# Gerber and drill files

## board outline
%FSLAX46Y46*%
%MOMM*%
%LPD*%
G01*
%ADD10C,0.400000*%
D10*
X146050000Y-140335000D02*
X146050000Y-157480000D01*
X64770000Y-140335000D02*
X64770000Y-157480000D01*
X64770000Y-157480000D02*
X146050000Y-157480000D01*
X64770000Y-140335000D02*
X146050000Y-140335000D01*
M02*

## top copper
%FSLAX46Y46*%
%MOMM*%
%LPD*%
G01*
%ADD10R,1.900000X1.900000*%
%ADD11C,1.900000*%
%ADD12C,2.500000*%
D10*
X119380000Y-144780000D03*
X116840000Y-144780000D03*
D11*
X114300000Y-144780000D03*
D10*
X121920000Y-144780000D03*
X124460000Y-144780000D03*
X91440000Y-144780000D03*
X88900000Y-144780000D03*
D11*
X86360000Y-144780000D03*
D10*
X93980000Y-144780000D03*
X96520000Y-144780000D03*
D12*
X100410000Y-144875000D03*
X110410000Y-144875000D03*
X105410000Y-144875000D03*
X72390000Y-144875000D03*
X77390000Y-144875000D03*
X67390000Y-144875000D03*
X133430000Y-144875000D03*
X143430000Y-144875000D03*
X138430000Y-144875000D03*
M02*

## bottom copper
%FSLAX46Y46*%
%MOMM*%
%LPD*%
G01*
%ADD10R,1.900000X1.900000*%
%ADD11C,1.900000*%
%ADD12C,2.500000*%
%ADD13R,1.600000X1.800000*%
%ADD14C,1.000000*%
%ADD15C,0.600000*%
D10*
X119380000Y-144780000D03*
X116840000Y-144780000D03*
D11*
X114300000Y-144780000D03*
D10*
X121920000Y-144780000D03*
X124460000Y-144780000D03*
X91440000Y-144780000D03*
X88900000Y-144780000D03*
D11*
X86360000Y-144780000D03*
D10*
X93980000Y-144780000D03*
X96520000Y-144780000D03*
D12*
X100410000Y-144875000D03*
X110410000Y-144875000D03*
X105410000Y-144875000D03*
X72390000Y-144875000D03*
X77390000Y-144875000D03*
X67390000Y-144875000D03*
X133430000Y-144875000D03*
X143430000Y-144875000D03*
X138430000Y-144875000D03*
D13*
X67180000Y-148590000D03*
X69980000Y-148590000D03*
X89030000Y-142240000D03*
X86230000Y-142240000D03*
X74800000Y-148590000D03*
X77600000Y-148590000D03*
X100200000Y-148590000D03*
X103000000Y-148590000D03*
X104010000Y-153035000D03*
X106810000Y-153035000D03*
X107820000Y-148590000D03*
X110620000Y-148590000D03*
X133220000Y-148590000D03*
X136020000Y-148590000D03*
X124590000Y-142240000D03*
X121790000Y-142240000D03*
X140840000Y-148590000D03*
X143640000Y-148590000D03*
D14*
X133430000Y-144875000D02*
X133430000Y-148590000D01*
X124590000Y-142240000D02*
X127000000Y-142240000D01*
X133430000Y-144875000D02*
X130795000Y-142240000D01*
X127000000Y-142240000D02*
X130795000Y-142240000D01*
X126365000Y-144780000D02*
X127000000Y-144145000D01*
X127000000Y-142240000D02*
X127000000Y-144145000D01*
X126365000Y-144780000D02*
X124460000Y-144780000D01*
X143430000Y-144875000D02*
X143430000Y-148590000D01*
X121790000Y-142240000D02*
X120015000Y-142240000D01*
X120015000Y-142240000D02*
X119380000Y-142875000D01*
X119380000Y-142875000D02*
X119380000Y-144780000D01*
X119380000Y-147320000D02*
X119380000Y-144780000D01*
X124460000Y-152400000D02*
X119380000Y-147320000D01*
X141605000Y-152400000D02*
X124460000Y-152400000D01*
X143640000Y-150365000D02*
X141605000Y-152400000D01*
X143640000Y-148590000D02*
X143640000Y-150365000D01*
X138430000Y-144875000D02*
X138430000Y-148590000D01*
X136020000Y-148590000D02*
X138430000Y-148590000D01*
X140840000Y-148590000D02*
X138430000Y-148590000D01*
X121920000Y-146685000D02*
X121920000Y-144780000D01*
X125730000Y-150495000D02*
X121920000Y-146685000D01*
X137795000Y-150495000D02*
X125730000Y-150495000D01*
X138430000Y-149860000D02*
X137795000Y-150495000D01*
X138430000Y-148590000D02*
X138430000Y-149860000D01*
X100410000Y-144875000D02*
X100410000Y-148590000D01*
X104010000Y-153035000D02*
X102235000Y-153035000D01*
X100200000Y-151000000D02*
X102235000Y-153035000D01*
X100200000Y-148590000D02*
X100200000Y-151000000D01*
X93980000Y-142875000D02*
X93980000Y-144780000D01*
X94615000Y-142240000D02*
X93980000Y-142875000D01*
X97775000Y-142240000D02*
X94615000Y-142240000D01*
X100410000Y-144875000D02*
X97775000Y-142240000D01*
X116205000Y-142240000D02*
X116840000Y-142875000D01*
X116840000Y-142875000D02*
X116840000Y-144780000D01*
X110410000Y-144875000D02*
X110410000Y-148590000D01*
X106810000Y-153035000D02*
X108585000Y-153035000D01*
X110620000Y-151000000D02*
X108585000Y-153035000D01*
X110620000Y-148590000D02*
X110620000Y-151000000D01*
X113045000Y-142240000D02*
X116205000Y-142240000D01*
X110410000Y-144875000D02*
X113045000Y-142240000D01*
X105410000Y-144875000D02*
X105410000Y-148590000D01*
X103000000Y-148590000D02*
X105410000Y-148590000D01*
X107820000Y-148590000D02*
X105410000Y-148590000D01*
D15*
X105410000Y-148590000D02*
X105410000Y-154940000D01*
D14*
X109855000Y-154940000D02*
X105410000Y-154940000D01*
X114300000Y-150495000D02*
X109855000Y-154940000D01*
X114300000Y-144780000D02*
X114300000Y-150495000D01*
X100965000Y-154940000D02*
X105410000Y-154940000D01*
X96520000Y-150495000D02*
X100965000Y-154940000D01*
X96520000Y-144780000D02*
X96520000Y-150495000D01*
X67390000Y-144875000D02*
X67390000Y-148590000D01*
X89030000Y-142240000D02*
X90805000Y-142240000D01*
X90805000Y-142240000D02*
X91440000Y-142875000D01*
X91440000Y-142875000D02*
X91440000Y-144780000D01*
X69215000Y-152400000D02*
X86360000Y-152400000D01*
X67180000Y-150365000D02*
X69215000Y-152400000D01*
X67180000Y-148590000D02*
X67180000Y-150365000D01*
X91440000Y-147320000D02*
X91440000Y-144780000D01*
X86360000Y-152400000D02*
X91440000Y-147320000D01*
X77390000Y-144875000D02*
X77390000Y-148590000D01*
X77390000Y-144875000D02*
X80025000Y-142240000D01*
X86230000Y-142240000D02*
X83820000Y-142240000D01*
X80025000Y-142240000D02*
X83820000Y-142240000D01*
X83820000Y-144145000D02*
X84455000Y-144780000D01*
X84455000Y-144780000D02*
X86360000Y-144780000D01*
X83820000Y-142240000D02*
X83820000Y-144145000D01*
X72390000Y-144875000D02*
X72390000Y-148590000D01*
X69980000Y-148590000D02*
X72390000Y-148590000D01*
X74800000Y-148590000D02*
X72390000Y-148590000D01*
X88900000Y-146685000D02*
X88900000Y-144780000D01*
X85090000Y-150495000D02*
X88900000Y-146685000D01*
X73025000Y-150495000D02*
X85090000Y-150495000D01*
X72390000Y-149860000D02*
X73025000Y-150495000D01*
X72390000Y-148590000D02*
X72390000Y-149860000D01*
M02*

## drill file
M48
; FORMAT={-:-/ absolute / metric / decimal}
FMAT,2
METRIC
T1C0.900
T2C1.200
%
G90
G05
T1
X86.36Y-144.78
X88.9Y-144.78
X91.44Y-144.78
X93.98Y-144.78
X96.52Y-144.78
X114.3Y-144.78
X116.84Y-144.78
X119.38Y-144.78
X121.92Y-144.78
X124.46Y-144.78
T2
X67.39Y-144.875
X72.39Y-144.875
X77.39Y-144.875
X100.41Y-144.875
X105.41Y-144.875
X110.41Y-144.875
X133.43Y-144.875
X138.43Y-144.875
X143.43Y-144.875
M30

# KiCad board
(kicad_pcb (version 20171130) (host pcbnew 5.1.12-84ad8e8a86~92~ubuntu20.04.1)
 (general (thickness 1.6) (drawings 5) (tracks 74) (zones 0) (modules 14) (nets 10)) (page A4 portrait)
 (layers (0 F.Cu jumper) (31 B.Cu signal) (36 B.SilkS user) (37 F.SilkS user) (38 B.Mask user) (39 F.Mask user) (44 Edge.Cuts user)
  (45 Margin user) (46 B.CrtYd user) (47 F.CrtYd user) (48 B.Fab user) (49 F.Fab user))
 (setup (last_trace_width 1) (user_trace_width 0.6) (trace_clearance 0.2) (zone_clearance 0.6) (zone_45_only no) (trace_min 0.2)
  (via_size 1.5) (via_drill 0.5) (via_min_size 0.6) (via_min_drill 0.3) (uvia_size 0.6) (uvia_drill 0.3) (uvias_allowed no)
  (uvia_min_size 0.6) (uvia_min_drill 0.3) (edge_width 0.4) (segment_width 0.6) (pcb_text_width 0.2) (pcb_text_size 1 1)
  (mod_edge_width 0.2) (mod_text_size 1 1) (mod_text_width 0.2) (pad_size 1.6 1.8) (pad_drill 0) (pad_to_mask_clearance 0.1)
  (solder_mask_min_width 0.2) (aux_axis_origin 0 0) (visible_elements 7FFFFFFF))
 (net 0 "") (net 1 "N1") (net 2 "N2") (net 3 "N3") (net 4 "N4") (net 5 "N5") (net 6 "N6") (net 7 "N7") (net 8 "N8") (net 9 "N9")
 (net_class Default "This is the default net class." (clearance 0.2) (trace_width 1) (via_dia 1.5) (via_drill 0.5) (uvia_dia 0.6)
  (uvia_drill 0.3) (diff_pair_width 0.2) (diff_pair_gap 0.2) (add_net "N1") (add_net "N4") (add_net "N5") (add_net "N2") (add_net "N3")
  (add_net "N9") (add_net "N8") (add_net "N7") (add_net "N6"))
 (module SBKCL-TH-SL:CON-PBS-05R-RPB (layer F.Cu) (at 119.38 144.78)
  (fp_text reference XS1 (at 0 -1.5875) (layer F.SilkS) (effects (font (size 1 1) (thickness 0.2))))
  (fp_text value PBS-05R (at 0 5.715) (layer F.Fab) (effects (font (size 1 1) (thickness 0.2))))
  (pad 3 thru_hole rect (at 0 0) (size 1.9 1.9) (drill 0.9) (layers B.Cu B.Mask) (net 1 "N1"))
  (pad 2 thru_hole rect (at -2.54 0) (size 1.9 1.9) (drill 0.9) (layers B.Cu B.Mask) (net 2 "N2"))
  (pad 1 thru_hole circle (at -5.08 0) (size 1.9 1.9) (drill 0.9) (layers B.Cu B.Mask) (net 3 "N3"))
  (pad 4 thru_hole rect (at 2.54 0) (size 1.9 1.9) (drill 0.9) (layers B.Cu B.Mask) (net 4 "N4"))
  (pad 5 thru_hole rect (at 5.08 0) (size 1.9 1.9) (drill 0.9) (layers B.Cu B.Mask) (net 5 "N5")))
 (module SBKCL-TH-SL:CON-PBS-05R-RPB (layer F.Cu) (at 91.44 144.78)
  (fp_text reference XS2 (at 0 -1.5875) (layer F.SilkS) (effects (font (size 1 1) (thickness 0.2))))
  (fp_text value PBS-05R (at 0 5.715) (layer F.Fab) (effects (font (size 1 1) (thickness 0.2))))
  (pad 3 thru_hole rect (at 0 0) (size 1.9 1.9) (drill 0.9) (layers B.Cu B.Mask) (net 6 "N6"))
  (pad 2 thru_hole rect (at -2.54 0) (size 1.9 1.9) (drill 0.9) (layers B.Cu B.Mask) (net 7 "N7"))
  (pad 1 thru_hole circle (at -5.08 0) (size 1.9 1.9) (drill 0.9) (layers B.Cu B.Mask) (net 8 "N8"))
  (pad 4 thru_hole rect (at 2.54 0) (size 1.9 1.9) (drill 0.9) (layers B.Cu B.Mask) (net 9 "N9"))
  (pad 5 thru_hole rect (at 5.08 0) (size 1.9 1.9) (drill 0.9) (layers B.Cu B.Mask) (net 3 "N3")))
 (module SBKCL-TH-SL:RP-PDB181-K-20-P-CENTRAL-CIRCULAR (layer F.Cu) (at 105.41 144.875 180)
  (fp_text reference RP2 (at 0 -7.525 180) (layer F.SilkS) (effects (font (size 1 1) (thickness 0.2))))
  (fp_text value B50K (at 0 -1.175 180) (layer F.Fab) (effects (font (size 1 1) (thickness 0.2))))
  (pad 3 thru_hole circle (at 5 0 180) (size 2.5 2.5) (drill 1.2) (layers B.Cu B.Mask) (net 9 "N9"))
  (pad 1 thru_hole circle (at -5 0 180) (size 2.5 2.5) (drill 1.2) (layers B.Cu B.Mask) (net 2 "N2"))
  (pad 2 thru_hole circle (at 0 0 180) (size 2.5 2.5) (drill 1.2) (layers B.Cu B.Mask) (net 3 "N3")))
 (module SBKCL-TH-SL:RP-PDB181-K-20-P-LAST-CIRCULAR (layer F.Cu) (at 72.39 144.875 180)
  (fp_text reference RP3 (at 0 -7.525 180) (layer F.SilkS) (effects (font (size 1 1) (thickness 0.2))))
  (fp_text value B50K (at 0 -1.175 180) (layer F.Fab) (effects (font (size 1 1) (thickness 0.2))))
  (pad 2 thru_hole circle (at 0 0 180) (size 2.5 2.5) (drill 1.2) (layers B.Cu B.Mask) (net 7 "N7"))
  (pad 1 thru_hole circle (at -5 0 180) (size 2.5 2.5) (drill 1.2) (layers B.Cu B.Mask) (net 8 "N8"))
  (pad 3 thru_hole circle (at 5 0 180) (size 2.5 2.5) (drill 1.2) (layers B.Cu B.Mask) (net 6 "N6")))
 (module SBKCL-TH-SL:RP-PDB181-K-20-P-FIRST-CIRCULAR (layer F.Cu) (at 138.43 144.875 180)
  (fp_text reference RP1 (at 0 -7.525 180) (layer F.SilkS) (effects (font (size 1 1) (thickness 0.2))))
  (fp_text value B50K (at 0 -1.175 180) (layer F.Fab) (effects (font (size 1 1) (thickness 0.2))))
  (pad 3 thru_hole circle (at 5 0 180) (size 2.5 2.5) (drill 1.2) (layers B.Cu B.Mask) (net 5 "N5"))
  (pad 1 thru_hole circle (at -5 0 180) (size 2.5 2.5) (drill 1.2) (layers B.Cu B.Mask) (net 1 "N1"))
  (pad 2 thru_hole circle (at 0 0 180) (size 2.5 2.5) (drill 1.2) (layers B.Cu B.Mask) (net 4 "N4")))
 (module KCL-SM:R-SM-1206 (layer B.Cu) (at 68.58 148.59)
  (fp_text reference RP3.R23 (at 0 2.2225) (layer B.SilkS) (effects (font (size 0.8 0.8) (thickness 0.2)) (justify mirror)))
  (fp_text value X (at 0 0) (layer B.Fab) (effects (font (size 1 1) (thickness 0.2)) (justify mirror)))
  (pad 1 smd rect (at -1.4 0) (size 1.6 1.8) (layers B.Cu B.Mask) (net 6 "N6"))
  (pad 2 smd rect (at 1.4 0) (size 1.6 1.8) (layers B.Cu B.Mask) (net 7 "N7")))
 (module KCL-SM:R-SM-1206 (layer B.Cu) (at 87.63 142.24 180)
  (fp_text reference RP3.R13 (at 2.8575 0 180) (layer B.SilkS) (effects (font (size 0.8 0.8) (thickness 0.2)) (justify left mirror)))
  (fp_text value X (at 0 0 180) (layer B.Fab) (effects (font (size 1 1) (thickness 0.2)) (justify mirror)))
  (pad 1 smd rect (at -1.4 0 180) (size 1.6 1.8) (layers B.Cu B.Mask) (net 6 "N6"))
  (pad 2 smd rect (at 1.4 0 180) (size 1.6 1.8) (layers B.Cu B.Mask) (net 8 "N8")))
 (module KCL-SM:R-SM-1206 (layer B.Cu) (at 76.2 148.59)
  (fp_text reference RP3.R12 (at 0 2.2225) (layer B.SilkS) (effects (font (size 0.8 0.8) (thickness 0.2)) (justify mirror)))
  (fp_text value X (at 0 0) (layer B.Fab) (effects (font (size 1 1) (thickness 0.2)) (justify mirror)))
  (pad 1 smd rect (at -1.4 0) (size 1.6 1.8) (layers B.Cu B.Mask) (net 7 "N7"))
  (pad 2 smd rect (at 1.4 0) (size 1.6 1.8) (layers B.Cu B.Mask) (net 8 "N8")))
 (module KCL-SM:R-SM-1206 (layer B.Cu) (at 101.6 148.59)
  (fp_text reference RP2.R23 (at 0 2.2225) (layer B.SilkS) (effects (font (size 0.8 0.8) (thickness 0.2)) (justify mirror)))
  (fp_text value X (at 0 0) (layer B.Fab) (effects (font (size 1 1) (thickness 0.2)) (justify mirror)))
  (pad 1 smd rect (at -1.4 0) (size 1.6 1.8) (layers B.Cu B.Mask) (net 9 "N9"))
  (pad 2 smd rect (at 1.4 0) (size 1.6 1.8) (layers B.Cu B.Mask) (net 3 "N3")))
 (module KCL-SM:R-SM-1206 (layer B.Cu) (at 105.41 153.035)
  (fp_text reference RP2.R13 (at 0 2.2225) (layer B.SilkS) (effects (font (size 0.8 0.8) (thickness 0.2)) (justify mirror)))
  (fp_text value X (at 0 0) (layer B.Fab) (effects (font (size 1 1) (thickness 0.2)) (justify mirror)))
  (pad 1 smd rect (at -1.4 0) (size 1.6 1.8) (layers B.Cu B.Mask) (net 9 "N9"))
  (pad 2 smd rect (at 1.4 0) (size 1.6 1.8) (layers B.Cu B.Mask) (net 2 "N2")))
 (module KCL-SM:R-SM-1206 (layer B.Cu) (at 109.22 148.59)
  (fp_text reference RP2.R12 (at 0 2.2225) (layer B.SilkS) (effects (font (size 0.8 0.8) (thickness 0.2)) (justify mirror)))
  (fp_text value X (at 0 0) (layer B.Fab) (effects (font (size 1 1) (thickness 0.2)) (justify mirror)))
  (pad 1 smd rect (at -1.4 0) (size 1.6 1.8) (layers B.Cu B.Mask) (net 3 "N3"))
  (pad 2 smd rect (at 1.4 0) (size 1.6 1.8) (layers B.Cu B.Mask) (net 2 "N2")))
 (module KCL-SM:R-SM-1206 (layer B.Cu) (at 134.62 148.59)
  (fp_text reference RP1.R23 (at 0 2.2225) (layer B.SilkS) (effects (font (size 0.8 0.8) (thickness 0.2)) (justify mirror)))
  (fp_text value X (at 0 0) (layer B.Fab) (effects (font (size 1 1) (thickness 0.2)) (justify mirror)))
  (pad 1 smd rect (at -1.4 0) (size 1.6 1.8) (layers B.Cu B.Mask) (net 5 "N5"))
  (pad 2 smd rect (at 1.4 0) (size 1.6 1.8) (layers B.Cu B.Mask) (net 4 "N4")))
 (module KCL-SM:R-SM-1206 (layer B.Cu) (at 123.19 142.24 180)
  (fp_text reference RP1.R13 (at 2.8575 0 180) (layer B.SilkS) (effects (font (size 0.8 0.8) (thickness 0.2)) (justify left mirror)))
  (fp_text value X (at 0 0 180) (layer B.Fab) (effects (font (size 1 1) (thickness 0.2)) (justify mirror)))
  (pad 1 smd rect (at -1.4 0 180) (size 1.6 1.8) (layers B.Cu B.Mask) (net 5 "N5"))
  (pad 2 smd rect (at 1.4 0 180) (size 1.6 1.8) (layers B.Cu B.Mask) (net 1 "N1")))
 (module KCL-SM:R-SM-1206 (layer B.Cu) (at 142.24 148.59)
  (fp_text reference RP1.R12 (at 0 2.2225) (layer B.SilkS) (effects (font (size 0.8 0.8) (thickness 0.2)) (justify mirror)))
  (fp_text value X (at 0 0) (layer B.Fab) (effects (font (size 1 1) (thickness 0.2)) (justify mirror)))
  (pad 1 smd rect (at -1.4 0) (size 1.6 1.8) (layers B.Cu B.Mask) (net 4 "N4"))
  (pad 2 smd rect (at 1.4 0) (size 1.6 1.8) (layers B.Cu B.Mask) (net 1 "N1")))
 (gr_line (start 146.05 140.335) (end 146.05 157.48) (layer Edge.Cuts) (width 0.4))
 (gr_line (start 64.77 140.335) (end 64.77 157.48) (layer Edge.Cuts) (width 0.4))
 (gr_line (start 64.77 157.48) (end 146.05 157.48) (layer Edge.Cuts) (width 0.4))
 (gr_line (start 64.77 140.335) (end 146.05 140.335) (layer Edge.Cuts) (width 0.4))
 (segment (start 133.43 144.875) (end 133.43 148.59) (width 1) (layer B.Cu) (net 5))
 (segment (start 124.59 142.24) (end 127 142.24) (width 1) (layer B.Cu) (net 5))
 (segment (start 133.43 144.875) (end 130.795 142.24) (width 1) (layer B.Cu) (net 5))
 (segment (start 127 142.24) (end 130.795 142.24) (width 1) (layer B.Cu) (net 5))
 (segment (start 126.365 144.78) (end 127 144.145) (width 1) (layer B.Cu) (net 5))
 (segment (start 127 142.24) (end 127 144.145) (width 1) (layer B.Cu) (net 5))
 (segment (start 126.365 144.78) (end 124.46 144.78) (width 1) (layer B.Cu) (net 5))
 (segment (start 143.43 144.875) (end 143.43 148.59) (width 1) (layer B.Cu) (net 1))
 (segment (start 121.79 142.24) (end 120.015 142.24) (width 1) (layer B.Cu) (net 1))
 (segment (start 120.015 142.24) (end 119.38 142.875) (width 1) (layer B.Cu) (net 1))
 (segment (start 119.38 142.875) (end 119.38 144.78) (width 1) (layer B.Cu) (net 1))
 (segment (start 119.38 147.32) (end 119.38 144.78) (width 1) (layer B.Cu) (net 1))
 (segment (start 124.46 152.4) (end 119.38 147.32) (width 1) (layer B.Cu) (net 1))
 (segment (start 141.605 152.4) (end 124.46 152.4) (width 1) (layer B.Cu) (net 1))
 (segment (start 143.64 150.365) (end 141.605 152.4) (width 1) (layer B.Cu) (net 1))
 (segment (start 143.64 148.59) (end 143.64 150.365) (width 1) (layer B.Cu) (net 1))
 (segment (start 138.43 144.875) (end 138.43 148.59) (width 1) (layer B.Cu) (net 4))
 (segment (start 136.02 148.59) (end 138.43 148.59) (width 1) (layer B.Cu) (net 4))
 (segment (start 140.84 148.59) (end 138.43 148.59) (width 1) (layer B.Cu) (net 4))
 (segment (start 121.92 146.685) (end 121.92 144.78) (width 1) (layer B.Cu) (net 4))
 (segment (start 125.73 150.495) (end 121.92 146.685) (width 1) (layer B.Cu) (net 4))
 (segment (start 137.795 150.495) (end 125.73 150.495) (width 1) (layer B.Cu) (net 4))
 (segment (start 138.43 149.86) (end 137.795 150.495) (width 1) (layer B.Cu) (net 4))
 (segment (start 138.43 148.59) (end 138.43 149.86) (width 1) (layer B.Cu) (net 4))
 (segment (start 100.41 144.875) (end 100.41 148.59) (width 1) (layer B.Cu) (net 9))
 (segment (start 104.01 153.035) (end 102.235 153.035) (width 1) (layer B.Cu) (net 9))
 (segment (start 100.2 151) (end 102.235 153.035) (width 1) (layer B.Cu) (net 9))
 (segment (start 100.2 148.59) (end 100.2 151) (width 1) (layer B.Cu) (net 9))
 (segment (start 93.98 142.875) (end 93.98 144.78) (width 1) (layer B.Cu) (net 9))
 (segment (start 94.615 142.24) (end 93.98 142.875) (width 1) (layer B.Cu) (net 9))
 (segment (start 97.775 142.24) (end 94.615 142.24) (width 1) (layer B.Cu) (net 9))
 (segment (start 100.41 144.875) (end 97.775 142.24) (width 1) (layer B.Cu) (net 9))
 (segment (start 116.205 142.24) (end 116.84 142.875) (width 1) (layer B.Cu) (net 2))
 (segment (start 116.84 142.875) (end 116.84 144.78) (width 1) (layer B.Cu) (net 2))
 (segment (start 110.41 144.875) (end 110.41 148.59) (width 1) (layer B.Cu) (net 2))
 (segment (start 106.81 153.035) (end 108.585 153.035) (width 1) (layer B.Cu) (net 2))
 (segment (start 110.62 151) (end 108.585 153.035) (width 1) (layer B.Cu) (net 2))
 (segment (start 110.62 148.59) (end 110.62 151) (width 1) (layer B.Cu) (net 2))
 (segment (start 113.045 142.24) (end 116.205 142.24) (width 1) (layer B.Cu) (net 2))
 (segment (start 110.41 144.875) (end 113.045 142.24) (width 1) (layer B.Cu) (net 2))
 (segment (start 105.41 144.875) (end 105.41 148.59) (width 1) (layer B.Cu) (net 3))
 (segment (start 103 148.59) (end 105.41 148.59) (width 1) (layer B.Cu) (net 3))
 (segment (start 107.82 148.59) (end 105.41 148.59) (width 1) (layer B.Cu) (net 3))
 (segment (start 105.41 148.59) (end 105.41 154.94) (width 0.6) (layer B.Cu) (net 3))
 (segment (start 109.855 154.94) (end 105.41 154.94) (width 1) (layer B.Cu) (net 3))
 (segment (start 114.3 150.495) (end 109.855 154.94) (width 1) (layer B.Cu) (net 3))
 (segment (start 114.3 144.78) (end 114.3 150.495) (width 1) (layer B.Cu) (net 3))
 (segment (start 100.965 154.94) (end 105.41 154.94) (width 1) (layer B.Cu) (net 3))
 (segment (start 96.52 150.495) (end 100.965 154.94) (width 1) (layer B.Cu) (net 3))
 (segment (start 96.52 144.78) (end 96.52 150.495) (width 1) (layer B.Cu) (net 3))
 (segment (start 67.39 144.875) (end 67.39 148.59) (width 1) (layer B.Cu) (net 6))
 (segment (start 89.03 142.24) (end 90.805 142.24) (width 1) (layer B.Cu) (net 6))
 (segment (start 90.805 142.24) (end 91.44 142.875) (width 1) (layer B.Cu) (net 6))
 (segment (start 91.44 142.875) (end 91.44 144.78) (width 1) (layer B.Cu) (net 6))
 (segment (start 69.215 152.4) (end 86.36 152.4) (width 1) (layer B.Cu) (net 6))
 (segment (start 67.18 150.365) (end 69.215 152.4) (width 1) (layer B.Cu) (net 6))
 (segment (start 67.18 148.59) (end 67.18 150.365) (width 1) (layer B.Cu) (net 6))
 (segment (start 91.44 147.32) (end 91.44 144.78) (width 1) (layer B.Cu) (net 6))
 (segment (start 86.36 152.4) (end 91.44 147.32) (width 1) (layer B.Cu) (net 6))
 (segment (start 77.39 144.875) (end 77.39 148.59) (width 1) (layer B.Cu) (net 8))
 (segment (start 77.39 144.875) (end 80.025 142.24) (width 1) (layer B.Cu) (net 8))
 (segment (start 86.23 142.24) (end 83.82 142.24) (width 1) (layer B.Cu) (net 8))
 (segment (start 80.025 142.24) (end 83.82 142.24) (width 1) (layer B.Cu) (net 8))
 (segment (start 83.82 144.145) (end 84.455 144.78) (width 1) (layer B.Cu) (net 8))
 (segment (start 84.455 144.78) (end 86.36 144.78) (width 1) (layer B.Cu) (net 8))
 (segment (start 83.82 142.24) (end 83.82 144.145) (width 1) (layer B.Cu) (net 8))
 (segment (start 72.39 144.875) (end 72.39 148.59) (width 1) (layer B.Cu) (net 7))
 (segment (start 69.98 148.59) (end 72.39 148.59) (width 1) (layer B.Cu) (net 7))
 (segment (start 74.8 148.59) (end 72.39 148.59) (width 1) (layer B.Cu) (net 7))
 (segment (start 88.9 146.685) (end 88.9 144.78) (width 1) (layer B.Cu) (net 7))
 (segment (start 85.09 150.495) (end 88.9 146.685) (width 1) (layer B.Cu) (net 7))
 (segment (start 73.025 150.495) (end 85.09 150.495) (width 1) (layer B.Cu) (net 7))
 (segment (start 72.39 149.86) (end 73.025 150.495) (width 1) (layer B.Cu) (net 7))
 (segment (start 72.39 148.59) (end 72.39 149.86) (width 1) (layer B.Cu) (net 7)))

